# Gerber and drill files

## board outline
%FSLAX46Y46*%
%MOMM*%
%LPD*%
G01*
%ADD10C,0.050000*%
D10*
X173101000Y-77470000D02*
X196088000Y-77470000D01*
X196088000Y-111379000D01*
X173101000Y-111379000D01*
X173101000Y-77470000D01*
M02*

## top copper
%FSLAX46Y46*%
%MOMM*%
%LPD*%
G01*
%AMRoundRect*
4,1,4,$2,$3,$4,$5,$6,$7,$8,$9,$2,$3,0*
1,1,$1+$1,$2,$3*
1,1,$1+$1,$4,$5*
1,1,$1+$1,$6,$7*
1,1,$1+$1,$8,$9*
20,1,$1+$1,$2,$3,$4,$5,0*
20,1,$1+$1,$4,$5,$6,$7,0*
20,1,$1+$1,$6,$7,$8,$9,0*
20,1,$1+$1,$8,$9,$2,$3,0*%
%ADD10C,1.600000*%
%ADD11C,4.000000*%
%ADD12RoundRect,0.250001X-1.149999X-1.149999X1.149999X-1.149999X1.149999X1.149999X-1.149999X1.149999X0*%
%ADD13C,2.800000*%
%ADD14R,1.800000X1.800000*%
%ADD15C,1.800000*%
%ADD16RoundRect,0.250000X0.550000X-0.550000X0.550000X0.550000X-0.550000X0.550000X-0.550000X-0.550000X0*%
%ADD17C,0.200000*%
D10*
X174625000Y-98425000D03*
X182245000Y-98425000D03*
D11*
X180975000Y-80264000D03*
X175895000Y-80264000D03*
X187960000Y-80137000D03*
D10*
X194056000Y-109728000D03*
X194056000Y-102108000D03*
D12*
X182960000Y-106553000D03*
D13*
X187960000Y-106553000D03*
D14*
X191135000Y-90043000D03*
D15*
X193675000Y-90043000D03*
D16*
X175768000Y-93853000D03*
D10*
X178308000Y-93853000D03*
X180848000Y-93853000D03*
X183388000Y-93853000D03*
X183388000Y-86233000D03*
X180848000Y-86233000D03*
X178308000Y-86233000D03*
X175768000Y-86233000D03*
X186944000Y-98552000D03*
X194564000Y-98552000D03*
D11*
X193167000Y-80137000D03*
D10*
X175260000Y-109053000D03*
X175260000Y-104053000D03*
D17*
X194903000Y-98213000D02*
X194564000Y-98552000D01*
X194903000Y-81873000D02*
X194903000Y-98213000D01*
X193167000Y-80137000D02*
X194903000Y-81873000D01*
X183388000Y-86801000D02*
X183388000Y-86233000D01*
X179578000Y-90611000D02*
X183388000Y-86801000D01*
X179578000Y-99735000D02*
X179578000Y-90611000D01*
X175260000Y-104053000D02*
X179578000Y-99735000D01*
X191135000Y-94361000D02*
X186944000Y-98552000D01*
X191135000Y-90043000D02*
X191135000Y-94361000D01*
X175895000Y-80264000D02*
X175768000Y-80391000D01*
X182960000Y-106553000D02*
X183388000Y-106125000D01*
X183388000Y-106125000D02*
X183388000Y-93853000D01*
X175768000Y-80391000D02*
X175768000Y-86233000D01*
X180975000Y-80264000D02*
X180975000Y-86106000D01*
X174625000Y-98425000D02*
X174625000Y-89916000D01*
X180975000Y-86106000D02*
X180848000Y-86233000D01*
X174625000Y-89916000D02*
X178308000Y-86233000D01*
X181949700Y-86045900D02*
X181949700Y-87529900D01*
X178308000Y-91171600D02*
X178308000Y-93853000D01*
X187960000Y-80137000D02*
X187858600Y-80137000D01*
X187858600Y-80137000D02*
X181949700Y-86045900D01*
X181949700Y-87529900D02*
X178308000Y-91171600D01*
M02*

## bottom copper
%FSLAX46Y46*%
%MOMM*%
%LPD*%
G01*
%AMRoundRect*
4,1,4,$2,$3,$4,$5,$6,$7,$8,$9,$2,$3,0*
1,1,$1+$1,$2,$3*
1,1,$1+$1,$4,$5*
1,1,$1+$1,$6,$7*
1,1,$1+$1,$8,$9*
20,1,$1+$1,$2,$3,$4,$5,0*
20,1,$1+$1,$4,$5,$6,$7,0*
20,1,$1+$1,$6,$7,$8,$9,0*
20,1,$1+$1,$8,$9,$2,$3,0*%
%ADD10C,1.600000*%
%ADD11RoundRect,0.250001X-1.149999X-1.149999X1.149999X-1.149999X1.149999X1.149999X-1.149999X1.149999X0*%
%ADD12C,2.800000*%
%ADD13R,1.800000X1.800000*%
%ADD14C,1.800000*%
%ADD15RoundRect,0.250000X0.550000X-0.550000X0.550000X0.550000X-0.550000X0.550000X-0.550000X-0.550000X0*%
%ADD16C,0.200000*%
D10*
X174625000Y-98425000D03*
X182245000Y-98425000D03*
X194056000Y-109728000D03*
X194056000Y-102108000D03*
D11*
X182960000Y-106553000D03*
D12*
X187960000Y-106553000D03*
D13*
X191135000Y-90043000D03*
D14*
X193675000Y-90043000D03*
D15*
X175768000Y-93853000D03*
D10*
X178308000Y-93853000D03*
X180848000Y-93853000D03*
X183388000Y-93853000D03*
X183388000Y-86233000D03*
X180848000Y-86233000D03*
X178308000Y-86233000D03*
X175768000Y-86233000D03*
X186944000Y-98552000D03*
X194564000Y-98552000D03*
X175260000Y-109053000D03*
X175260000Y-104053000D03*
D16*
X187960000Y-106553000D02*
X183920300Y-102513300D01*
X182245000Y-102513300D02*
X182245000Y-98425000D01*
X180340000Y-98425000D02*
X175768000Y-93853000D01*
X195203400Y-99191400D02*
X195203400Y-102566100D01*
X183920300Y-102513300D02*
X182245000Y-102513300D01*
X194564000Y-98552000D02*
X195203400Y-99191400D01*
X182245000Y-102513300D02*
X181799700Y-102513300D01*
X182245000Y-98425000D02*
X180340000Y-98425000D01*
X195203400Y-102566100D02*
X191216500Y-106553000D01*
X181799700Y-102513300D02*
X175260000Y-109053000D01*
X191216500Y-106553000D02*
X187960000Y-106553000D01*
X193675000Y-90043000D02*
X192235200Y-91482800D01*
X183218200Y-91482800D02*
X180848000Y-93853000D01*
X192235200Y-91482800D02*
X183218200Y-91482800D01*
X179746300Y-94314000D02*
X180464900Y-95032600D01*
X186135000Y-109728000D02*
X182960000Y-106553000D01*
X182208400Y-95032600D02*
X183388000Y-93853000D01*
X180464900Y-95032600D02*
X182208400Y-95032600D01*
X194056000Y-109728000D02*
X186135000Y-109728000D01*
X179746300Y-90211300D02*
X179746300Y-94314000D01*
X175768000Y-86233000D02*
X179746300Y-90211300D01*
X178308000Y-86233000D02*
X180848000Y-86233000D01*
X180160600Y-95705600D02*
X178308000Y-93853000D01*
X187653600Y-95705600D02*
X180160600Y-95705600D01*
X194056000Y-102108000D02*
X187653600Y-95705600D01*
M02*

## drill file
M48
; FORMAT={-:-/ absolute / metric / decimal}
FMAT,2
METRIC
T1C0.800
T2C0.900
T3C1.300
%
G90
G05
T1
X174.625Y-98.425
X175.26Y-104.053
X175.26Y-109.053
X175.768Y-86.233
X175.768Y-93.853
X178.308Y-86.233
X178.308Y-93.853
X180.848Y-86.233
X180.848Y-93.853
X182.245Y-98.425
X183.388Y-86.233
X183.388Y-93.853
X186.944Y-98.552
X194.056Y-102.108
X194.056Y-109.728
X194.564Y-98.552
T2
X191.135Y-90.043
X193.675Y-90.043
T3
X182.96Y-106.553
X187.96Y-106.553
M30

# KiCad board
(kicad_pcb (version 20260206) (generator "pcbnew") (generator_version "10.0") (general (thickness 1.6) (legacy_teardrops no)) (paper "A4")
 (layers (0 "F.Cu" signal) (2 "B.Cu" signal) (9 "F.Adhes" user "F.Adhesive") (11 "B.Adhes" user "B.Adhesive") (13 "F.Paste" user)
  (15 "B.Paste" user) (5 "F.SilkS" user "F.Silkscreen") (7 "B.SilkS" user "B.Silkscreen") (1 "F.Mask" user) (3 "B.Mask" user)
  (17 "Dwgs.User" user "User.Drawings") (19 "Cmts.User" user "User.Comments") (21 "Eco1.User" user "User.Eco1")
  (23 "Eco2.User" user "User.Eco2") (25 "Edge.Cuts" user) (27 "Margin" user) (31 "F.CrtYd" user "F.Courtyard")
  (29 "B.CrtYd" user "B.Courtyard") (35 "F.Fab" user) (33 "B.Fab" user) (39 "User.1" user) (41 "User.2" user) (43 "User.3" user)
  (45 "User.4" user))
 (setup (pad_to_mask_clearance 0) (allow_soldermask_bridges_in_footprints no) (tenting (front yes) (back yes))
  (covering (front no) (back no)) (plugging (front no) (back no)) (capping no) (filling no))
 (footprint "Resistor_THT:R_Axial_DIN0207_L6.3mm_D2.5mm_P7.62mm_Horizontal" (layer "F.Cu") (at 174.625 98.425)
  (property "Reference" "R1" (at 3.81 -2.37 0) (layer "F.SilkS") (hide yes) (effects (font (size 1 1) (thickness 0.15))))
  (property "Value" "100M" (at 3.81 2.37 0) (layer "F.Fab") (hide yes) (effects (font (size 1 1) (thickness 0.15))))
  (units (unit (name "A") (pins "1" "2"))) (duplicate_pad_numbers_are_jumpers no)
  (pad "1" thru_hole circle (at 0 0) (size 1.6 1.6) (drill 0.8) (layers "*.Cu" "*.Mask") (remove_unused_layers no) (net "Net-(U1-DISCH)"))
  (pad "2" thru_hole circle (at 7.62 0) (size 1.6 1.6) (drill 0.8) (layers "*.Cu" "*.Mask") (remove_unused_layers no) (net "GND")))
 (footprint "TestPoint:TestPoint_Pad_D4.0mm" (layer "F.Cu") (at 180.975 80.264 180)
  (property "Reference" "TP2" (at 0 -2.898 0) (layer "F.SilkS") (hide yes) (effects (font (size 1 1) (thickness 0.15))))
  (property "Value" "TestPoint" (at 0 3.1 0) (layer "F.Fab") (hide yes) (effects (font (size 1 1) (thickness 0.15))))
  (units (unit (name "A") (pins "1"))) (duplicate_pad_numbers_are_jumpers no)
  (pad "1" smd circle (at 0 0 180) (size 4 4) (layers "F.Cu" "F.Mask") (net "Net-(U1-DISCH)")))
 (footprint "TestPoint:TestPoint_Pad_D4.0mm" (layer "F.Cu") (at 175.895 80.264 180)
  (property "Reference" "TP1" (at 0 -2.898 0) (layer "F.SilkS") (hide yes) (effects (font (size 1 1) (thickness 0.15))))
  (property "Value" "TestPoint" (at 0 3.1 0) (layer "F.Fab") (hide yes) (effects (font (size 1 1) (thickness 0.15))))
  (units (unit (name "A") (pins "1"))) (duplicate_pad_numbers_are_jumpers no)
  (pad "1" smd circle (at 0 0 180) (size 4 4) (layers "F.Cu" "F.Mask") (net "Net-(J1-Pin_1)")))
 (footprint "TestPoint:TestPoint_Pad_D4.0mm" (layer "F.Cu") (at 187.96 80.137 180)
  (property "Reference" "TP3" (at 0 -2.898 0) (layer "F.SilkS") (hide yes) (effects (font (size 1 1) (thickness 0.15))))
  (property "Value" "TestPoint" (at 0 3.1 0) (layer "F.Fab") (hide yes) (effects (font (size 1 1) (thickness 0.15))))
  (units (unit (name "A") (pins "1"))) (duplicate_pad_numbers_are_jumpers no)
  (pad "1" smd circle (at 0 0 180) (size 4 4) (layers "F.Cu" "F.Mask") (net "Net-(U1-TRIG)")))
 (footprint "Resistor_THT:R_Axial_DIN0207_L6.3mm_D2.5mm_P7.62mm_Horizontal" (layer "F.Cu") (at 194.056 109.728 90)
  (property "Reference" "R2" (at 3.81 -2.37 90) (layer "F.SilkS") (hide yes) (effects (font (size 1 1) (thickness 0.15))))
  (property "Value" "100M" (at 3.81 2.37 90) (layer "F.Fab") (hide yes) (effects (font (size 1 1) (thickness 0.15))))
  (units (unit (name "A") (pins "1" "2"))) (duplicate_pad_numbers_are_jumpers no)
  (pad "1" thru_hole circle (at 0 0 90) (size 1.6 1.6) (drill 0.8) (layers "*.Cu" "*.Mask") (remove_unused_layers no) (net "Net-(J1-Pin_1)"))
  (pad "2" thru_hole circle (at 7.62 0 90) (size 1.6 1.6) (drill 0.8) (layers "*.Cu" "*.Mask") (remove_unused_layers no)
   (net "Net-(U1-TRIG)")))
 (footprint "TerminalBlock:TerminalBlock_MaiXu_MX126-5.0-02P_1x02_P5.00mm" (layer "F.Cu") (at 182.96 106.553)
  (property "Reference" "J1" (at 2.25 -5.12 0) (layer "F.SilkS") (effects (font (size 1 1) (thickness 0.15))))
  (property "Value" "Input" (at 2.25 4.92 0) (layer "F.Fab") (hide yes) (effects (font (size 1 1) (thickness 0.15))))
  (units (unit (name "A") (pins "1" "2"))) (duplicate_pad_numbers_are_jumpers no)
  (pad "1" thru_hole roundrect (at 0 0) (size 2.8 2.8) (drill 1.3) (layers "*.Cu" "*.Mask") (remove_unused_layers no)
   (roundrect_rratio 0.089286) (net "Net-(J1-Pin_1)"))
  (pad "2" thru_hole circle (at 5 0) (size 2.8 2.8) (drill 1.3) (layers "*.Cu" "*.Mask") (remove_unused_layers no) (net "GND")))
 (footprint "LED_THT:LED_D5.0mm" (layer "F.Cu") (at 191.135 90.043)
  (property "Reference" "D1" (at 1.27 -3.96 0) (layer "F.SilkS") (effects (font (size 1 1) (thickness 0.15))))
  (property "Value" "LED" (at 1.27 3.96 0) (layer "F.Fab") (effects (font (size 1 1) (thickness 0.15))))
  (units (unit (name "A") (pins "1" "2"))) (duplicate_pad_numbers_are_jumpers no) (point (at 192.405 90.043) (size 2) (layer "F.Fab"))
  (pad "1" thru_hole rect (at 0 0) (size 1.8 1.8) (drill 0.9) (layers "*.Cu" "*.Mask") (remove_unused_layers no) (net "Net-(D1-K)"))
  (pad "2" thru_hole circle (at 2.54 0) (size 1.8 1.8) (drill 0.9) (layers "*.Cu" "*.Mask") (remove_unused_layers no) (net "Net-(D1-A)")))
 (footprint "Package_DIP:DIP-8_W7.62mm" (layer "F.Cu") (at 175.768 93.853 90)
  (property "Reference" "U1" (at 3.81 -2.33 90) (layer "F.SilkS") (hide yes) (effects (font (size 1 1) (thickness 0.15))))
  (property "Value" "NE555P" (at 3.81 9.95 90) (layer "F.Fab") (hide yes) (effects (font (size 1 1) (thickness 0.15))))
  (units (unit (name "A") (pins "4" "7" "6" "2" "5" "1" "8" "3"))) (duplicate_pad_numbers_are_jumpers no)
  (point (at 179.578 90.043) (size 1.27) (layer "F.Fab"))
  (pad "1" thru_hole roundrect (at 0 0 90) (size 1.6 1.6) (drill 0.8) (layers "*.Cu" "*.Mask") (remove_unused_layers no)
   (roundrect_rratio 0.15625) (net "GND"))
  (pad "2" thru_hole circle (at 0 2.54 90) (size 1.6 1.6) (drill 0.8) (layers "*.Cu" "*.Mask") (remove_unused_layers no)
   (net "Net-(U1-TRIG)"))
  (pad "3" thru_hole circle (at 0 5.08 90) (size 1.6 1.6) (drill 0.8) (layers "*.Cu" "*.Mask") (remove_unused_layers no) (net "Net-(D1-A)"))
  (pad "4" thru_hole circle (at 0 7.62 90) (size 1.6 1.6) (drill 0.8) (layers "*.Cu" "*.Mask") (remove_unused_layers no)
   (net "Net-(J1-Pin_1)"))
  (pad "5" thru_hole circle (at 7.62 7.62 90) (size 1.6 1.6) (drill 0.8) (layers "*.Cu" "*.Mask") (remove_unused_layers no)
   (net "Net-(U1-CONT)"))
  (pad "6" thru_hole circle (at 7.62 5.08 90) (size 1.6 1.6) (drill 0.8) (layers "*.Cu" "*.Mask") (remove_unused_layers no)
   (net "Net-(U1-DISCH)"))
  (pad "7" thru_hole circle (at 7.62 2.54 90) (size 1.6 1.6) (drill 0.8) (layers "*.Cu" "*.Mask") (remove_unused_layers no)
   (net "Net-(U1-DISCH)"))
  (pad "8" thru_hole circle (at 7.62 0 90) (size 1.6 1.6) (drill 0.8) (layers "*.Cu" "*.Mask") (remove_unused_layers no)
   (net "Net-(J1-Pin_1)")))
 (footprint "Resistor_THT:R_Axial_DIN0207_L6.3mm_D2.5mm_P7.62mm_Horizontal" (layer "F.Cu") (at 186.944 98.552)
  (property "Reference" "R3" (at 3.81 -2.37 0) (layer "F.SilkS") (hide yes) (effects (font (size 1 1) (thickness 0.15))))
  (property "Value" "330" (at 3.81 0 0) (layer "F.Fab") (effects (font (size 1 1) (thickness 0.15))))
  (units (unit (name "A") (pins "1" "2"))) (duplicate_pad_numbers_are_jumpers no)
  (pad "1" thru_hole circle (at 0 0) (size 1.6 1.6) (drill 0.8) (layers "*.Cu" "*.Mask") (remove_unused_layers no) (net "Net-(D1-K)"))
  (pad "2" thru_hole circle (at 7.62 0) (size 1.6 1.6) (drill 0.8) (layers "*.Cu" "*.Mask") (remove_unused_layers no) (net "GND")))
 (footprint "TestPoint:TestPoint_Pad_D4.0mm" (layer "F.Cu") (at 193.167 80.137 180)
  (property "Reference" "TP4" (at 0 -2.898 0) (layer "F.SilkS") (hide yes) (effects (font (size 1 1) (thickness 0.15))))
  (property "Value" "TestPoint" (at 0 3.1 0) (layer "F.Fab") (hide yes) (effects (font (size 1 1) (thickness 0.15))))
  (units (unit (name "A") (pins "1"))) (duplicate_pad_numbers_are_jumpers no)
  (pad "1" smd circle (at 0 0 180) (size 4 4) (layers "F.Cu" "F.Mask") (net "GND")))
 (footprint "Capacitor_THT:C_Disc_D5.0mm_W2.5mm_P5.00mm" (layer "F.Cu") (at 175.26 109.053 90)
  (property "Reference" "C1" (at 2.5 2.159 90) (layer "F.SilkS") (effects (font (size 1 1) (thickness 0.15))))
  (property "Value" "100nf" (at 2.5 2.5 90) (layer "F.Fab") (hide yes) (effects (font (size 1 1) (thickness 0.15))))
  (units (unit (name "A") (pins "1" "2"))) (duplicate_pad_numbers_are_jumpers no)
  (pad "1" thru_hole circle (at 0 0 90) (size 1.6 1.6) (drill 0.8) (layers "*.Cu" "*.Mask") (remove_unused_layers no) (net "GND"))
  (pad "2" thru_hole circle (at 5 0 90) (size 1.6 1.6) (drill 0.8) (layers "*.Cu" "*.Mask") (remove_unused_layers no) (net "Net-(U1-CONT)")))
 (gr_rect (start 173.101 77.47) (end 196.088 111.379) (stroke (width 0.05) (type default)) (fill no) (layer "Edge.Cuts"))
 (segment (start 194.903 98.213) (end 194.564 98.552) (width 0.2) (layer "F.Cu") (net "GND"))
 (segment (start 194.903 81.873) (end 194.903 98.213) (width 0.2) (layer "F.Cu") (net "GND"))
 (segment (start 193.167 80.137) (end 194.903 81.873) (width 0.2) (layer "F.Cu") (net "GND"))
 (segment (start 187.96 106.553) (end 183.9203 102.5133) (width 0.2) (layer "B.Cu") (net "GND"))
 (segment (start 182.245 102.5133) (end 182.245 98.425) (width 0.2) (layer "B.Cu") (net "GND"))
 (segment (start 180.34 98.425) (end 175.768 93.853) (width 0.2) (layer "B.Cu") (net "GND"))
 (segment (start 195.2034 99.1914) (end 195.2034 102.5661) (width 0.2) (layer "B.Cu") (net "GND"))
 (segment (start 183.9203 102.5133) (end 182.245 102.5133) (width 0.2) (layer "B.Cu") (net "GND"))
 (segment (start 194.564 98.552) (end 195.2034 99.1914) (width 0.2) (layer "B.Cu") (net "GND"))
 (segment (start 182.245 102.5133) (end 181.7997 102.5133) (width 0.2) (layer "B.Cu") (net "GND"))
 (segment (start 182.245 98.425) (end 180.34 98.425) (width 0.2) (layer "B.Cu") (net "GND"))
 (segment (start 195.2034 102.5661) (end 191.2165 106.553) (width 0.2) (layer "B.Cu") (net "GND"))
 (segment (start 181.7997 102.5133) (end 175.26 109.053) (width 0.2) (layer "B.Cu") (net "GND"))
 (segment (start 191.2165 106.553) (end 187.96 106.553) (width 0.2) (layer "B.Cu") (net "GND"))
 (segment (start 183.388 86.801) (end 183.388 86.233) (width 0.2) (layer "F.Cu") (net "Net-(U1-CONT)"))
 (segment (start 179.578 90.611) (end 183.388 86.801) (width 0.2) (layer "F.Cu") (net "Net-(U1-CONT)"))
 (segment (start 179.578 99.735) (end 179.578 90.611) (width 0.2) (layer "F.Cu") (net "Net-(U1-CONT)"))
 (segment (start 175.26 104.053) (end 179.578 99.735) (width 0.2) (layer "F.Cu") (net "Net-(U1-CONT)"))
 (segment (start 193.675 90.043) (end 192.2352 91.4828) (width 0.2) (layer "B.Cu") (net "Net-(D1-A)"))
 (segment (start 183.2182 91.4828) (end 180.848 93.853) (width 0.2) (layer "B.Cu") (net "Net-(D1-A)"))
 (segment (start 192.2352 91.4828) (end 183.2182 91.4828) (width 0.2) (layer "B.Cu") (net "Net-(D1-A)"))
 (segment (start 191.135 94.361) (end 186.944 98.552) (width 0.2) (layer "F.Cu") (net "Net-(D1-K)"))
 (segment (start 191.135 90.043) (end 191.135 94.361) (width 0.2) (layer "F.Cu") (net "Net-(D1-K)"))
 (segment (start 175.895 80.264) (end 175.768 80.391) (width 0.2) (layer "F.Cu") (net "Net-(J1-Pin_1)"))
 (segment (start 182.96 106.553) (end 183.388 106.125) (width 0.2) (layer "F.Cu") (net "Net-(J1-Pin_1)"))
 (segment (start 183.388 106.125) (end 183.388 93.853) (width 0.2) (layer "F.Cu") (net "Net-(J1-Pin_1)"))
 (segment (start 175.768 80.391) (end 175.768 86.233) (width 0.2) (layer "F.Cu") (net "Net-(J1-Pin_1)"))
 (segment (start 179.7463 94.314) (end 180.4649 95.0326) (width 0.2) (layer "B.Cu") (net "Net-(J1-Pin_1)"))
 (segment (start 186.135 109.728) (end 182.96 106.553) (width 0.2) (layer "B.Cu") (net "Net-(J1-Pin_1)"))
 (segment (start 182.2084 95.0326) (end 183.388 93.853) (width 0.2) (layer "B.Cu") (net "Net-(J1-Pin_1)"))
 (segment (start 180.4649 95.0326) (end 182.2084 95.0326) (width 0.2) (layer "B.Cu") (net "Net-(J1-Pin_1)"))
 (segment (start 194.056 109.728) (end 186.135 109.728) (width 0.2) (layer "B.Cu") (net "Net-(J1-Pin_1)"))
 (segment (start 179.7463 90.2113) (end 179.7463 94.314) (width 0.2) (layer "B.Cu") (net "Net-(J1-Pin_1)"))
 (segment (start 175.768 86.233) (end 179.7463 90.2113) (width 0.2) (layer "B.Cu") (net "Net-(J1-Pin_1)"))
 (segment (start 180.975 80.264) (end 180.975 86.106) (width 0.2) (layer "F.Cu") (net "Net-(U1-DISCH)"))
 (segment (start 174.625 98.425) (end 174.625 89.916) (width 0.2) (layer "F.Cu") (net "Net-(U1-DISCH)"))
 (segment (start 180.975 86.106) (end 180.848 86.233) (width 0.2) (layer "F.Cu") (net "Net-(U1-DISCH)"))
 (segment (start 174.625 89.916) (end 178.308 86.233) (width 0.2) (layer "F.Cu") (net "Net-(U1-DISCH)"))
 (segment (start 178.308 86.233) (end 180.848 86.233) (width 0.2) (layer "B.Cu") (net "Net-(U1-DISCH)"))
 (segment (start 181.9497 86.0459) (end 181.9497 87.5299) (width 0.2) (layer "F.Cu") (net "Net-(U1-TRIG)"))
 (segment (start 178.308 91.1716) (end 178.308 93.853) (width 0.2) (layer "F.Cu") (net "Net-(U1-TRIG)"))
 (segment (start 187.96 80.137) (end 187.8586 80.137) (width 0.2) (layer "F.Cu") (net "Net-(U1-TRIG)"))
 (segment (start 187.8586 80.137) (end 181.9497 86.0459) (width 0.2) (layer "F.Cu") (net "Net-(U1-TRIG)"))
 (segment (start 181.9497 87.5299) (end 178.308 91.1716) (width 0.2) (layer "F.Cu") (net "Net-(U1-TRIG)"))
 (segment (start 180.1606 95.7056) (end 178.308 93.853) (width 0.2) (layer "B.Cu") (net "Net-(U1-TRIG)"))
 (segment (start 187.6536 95.7056) (end 180.1606 95.7056) (width 0.2) (layer "B.Cu") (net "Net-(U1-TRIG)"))
 (segment (start 194.056 102.108) (end 187.6536 95.7056) (width 0.2) (layer "B.Cu") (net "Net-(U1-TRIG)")))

